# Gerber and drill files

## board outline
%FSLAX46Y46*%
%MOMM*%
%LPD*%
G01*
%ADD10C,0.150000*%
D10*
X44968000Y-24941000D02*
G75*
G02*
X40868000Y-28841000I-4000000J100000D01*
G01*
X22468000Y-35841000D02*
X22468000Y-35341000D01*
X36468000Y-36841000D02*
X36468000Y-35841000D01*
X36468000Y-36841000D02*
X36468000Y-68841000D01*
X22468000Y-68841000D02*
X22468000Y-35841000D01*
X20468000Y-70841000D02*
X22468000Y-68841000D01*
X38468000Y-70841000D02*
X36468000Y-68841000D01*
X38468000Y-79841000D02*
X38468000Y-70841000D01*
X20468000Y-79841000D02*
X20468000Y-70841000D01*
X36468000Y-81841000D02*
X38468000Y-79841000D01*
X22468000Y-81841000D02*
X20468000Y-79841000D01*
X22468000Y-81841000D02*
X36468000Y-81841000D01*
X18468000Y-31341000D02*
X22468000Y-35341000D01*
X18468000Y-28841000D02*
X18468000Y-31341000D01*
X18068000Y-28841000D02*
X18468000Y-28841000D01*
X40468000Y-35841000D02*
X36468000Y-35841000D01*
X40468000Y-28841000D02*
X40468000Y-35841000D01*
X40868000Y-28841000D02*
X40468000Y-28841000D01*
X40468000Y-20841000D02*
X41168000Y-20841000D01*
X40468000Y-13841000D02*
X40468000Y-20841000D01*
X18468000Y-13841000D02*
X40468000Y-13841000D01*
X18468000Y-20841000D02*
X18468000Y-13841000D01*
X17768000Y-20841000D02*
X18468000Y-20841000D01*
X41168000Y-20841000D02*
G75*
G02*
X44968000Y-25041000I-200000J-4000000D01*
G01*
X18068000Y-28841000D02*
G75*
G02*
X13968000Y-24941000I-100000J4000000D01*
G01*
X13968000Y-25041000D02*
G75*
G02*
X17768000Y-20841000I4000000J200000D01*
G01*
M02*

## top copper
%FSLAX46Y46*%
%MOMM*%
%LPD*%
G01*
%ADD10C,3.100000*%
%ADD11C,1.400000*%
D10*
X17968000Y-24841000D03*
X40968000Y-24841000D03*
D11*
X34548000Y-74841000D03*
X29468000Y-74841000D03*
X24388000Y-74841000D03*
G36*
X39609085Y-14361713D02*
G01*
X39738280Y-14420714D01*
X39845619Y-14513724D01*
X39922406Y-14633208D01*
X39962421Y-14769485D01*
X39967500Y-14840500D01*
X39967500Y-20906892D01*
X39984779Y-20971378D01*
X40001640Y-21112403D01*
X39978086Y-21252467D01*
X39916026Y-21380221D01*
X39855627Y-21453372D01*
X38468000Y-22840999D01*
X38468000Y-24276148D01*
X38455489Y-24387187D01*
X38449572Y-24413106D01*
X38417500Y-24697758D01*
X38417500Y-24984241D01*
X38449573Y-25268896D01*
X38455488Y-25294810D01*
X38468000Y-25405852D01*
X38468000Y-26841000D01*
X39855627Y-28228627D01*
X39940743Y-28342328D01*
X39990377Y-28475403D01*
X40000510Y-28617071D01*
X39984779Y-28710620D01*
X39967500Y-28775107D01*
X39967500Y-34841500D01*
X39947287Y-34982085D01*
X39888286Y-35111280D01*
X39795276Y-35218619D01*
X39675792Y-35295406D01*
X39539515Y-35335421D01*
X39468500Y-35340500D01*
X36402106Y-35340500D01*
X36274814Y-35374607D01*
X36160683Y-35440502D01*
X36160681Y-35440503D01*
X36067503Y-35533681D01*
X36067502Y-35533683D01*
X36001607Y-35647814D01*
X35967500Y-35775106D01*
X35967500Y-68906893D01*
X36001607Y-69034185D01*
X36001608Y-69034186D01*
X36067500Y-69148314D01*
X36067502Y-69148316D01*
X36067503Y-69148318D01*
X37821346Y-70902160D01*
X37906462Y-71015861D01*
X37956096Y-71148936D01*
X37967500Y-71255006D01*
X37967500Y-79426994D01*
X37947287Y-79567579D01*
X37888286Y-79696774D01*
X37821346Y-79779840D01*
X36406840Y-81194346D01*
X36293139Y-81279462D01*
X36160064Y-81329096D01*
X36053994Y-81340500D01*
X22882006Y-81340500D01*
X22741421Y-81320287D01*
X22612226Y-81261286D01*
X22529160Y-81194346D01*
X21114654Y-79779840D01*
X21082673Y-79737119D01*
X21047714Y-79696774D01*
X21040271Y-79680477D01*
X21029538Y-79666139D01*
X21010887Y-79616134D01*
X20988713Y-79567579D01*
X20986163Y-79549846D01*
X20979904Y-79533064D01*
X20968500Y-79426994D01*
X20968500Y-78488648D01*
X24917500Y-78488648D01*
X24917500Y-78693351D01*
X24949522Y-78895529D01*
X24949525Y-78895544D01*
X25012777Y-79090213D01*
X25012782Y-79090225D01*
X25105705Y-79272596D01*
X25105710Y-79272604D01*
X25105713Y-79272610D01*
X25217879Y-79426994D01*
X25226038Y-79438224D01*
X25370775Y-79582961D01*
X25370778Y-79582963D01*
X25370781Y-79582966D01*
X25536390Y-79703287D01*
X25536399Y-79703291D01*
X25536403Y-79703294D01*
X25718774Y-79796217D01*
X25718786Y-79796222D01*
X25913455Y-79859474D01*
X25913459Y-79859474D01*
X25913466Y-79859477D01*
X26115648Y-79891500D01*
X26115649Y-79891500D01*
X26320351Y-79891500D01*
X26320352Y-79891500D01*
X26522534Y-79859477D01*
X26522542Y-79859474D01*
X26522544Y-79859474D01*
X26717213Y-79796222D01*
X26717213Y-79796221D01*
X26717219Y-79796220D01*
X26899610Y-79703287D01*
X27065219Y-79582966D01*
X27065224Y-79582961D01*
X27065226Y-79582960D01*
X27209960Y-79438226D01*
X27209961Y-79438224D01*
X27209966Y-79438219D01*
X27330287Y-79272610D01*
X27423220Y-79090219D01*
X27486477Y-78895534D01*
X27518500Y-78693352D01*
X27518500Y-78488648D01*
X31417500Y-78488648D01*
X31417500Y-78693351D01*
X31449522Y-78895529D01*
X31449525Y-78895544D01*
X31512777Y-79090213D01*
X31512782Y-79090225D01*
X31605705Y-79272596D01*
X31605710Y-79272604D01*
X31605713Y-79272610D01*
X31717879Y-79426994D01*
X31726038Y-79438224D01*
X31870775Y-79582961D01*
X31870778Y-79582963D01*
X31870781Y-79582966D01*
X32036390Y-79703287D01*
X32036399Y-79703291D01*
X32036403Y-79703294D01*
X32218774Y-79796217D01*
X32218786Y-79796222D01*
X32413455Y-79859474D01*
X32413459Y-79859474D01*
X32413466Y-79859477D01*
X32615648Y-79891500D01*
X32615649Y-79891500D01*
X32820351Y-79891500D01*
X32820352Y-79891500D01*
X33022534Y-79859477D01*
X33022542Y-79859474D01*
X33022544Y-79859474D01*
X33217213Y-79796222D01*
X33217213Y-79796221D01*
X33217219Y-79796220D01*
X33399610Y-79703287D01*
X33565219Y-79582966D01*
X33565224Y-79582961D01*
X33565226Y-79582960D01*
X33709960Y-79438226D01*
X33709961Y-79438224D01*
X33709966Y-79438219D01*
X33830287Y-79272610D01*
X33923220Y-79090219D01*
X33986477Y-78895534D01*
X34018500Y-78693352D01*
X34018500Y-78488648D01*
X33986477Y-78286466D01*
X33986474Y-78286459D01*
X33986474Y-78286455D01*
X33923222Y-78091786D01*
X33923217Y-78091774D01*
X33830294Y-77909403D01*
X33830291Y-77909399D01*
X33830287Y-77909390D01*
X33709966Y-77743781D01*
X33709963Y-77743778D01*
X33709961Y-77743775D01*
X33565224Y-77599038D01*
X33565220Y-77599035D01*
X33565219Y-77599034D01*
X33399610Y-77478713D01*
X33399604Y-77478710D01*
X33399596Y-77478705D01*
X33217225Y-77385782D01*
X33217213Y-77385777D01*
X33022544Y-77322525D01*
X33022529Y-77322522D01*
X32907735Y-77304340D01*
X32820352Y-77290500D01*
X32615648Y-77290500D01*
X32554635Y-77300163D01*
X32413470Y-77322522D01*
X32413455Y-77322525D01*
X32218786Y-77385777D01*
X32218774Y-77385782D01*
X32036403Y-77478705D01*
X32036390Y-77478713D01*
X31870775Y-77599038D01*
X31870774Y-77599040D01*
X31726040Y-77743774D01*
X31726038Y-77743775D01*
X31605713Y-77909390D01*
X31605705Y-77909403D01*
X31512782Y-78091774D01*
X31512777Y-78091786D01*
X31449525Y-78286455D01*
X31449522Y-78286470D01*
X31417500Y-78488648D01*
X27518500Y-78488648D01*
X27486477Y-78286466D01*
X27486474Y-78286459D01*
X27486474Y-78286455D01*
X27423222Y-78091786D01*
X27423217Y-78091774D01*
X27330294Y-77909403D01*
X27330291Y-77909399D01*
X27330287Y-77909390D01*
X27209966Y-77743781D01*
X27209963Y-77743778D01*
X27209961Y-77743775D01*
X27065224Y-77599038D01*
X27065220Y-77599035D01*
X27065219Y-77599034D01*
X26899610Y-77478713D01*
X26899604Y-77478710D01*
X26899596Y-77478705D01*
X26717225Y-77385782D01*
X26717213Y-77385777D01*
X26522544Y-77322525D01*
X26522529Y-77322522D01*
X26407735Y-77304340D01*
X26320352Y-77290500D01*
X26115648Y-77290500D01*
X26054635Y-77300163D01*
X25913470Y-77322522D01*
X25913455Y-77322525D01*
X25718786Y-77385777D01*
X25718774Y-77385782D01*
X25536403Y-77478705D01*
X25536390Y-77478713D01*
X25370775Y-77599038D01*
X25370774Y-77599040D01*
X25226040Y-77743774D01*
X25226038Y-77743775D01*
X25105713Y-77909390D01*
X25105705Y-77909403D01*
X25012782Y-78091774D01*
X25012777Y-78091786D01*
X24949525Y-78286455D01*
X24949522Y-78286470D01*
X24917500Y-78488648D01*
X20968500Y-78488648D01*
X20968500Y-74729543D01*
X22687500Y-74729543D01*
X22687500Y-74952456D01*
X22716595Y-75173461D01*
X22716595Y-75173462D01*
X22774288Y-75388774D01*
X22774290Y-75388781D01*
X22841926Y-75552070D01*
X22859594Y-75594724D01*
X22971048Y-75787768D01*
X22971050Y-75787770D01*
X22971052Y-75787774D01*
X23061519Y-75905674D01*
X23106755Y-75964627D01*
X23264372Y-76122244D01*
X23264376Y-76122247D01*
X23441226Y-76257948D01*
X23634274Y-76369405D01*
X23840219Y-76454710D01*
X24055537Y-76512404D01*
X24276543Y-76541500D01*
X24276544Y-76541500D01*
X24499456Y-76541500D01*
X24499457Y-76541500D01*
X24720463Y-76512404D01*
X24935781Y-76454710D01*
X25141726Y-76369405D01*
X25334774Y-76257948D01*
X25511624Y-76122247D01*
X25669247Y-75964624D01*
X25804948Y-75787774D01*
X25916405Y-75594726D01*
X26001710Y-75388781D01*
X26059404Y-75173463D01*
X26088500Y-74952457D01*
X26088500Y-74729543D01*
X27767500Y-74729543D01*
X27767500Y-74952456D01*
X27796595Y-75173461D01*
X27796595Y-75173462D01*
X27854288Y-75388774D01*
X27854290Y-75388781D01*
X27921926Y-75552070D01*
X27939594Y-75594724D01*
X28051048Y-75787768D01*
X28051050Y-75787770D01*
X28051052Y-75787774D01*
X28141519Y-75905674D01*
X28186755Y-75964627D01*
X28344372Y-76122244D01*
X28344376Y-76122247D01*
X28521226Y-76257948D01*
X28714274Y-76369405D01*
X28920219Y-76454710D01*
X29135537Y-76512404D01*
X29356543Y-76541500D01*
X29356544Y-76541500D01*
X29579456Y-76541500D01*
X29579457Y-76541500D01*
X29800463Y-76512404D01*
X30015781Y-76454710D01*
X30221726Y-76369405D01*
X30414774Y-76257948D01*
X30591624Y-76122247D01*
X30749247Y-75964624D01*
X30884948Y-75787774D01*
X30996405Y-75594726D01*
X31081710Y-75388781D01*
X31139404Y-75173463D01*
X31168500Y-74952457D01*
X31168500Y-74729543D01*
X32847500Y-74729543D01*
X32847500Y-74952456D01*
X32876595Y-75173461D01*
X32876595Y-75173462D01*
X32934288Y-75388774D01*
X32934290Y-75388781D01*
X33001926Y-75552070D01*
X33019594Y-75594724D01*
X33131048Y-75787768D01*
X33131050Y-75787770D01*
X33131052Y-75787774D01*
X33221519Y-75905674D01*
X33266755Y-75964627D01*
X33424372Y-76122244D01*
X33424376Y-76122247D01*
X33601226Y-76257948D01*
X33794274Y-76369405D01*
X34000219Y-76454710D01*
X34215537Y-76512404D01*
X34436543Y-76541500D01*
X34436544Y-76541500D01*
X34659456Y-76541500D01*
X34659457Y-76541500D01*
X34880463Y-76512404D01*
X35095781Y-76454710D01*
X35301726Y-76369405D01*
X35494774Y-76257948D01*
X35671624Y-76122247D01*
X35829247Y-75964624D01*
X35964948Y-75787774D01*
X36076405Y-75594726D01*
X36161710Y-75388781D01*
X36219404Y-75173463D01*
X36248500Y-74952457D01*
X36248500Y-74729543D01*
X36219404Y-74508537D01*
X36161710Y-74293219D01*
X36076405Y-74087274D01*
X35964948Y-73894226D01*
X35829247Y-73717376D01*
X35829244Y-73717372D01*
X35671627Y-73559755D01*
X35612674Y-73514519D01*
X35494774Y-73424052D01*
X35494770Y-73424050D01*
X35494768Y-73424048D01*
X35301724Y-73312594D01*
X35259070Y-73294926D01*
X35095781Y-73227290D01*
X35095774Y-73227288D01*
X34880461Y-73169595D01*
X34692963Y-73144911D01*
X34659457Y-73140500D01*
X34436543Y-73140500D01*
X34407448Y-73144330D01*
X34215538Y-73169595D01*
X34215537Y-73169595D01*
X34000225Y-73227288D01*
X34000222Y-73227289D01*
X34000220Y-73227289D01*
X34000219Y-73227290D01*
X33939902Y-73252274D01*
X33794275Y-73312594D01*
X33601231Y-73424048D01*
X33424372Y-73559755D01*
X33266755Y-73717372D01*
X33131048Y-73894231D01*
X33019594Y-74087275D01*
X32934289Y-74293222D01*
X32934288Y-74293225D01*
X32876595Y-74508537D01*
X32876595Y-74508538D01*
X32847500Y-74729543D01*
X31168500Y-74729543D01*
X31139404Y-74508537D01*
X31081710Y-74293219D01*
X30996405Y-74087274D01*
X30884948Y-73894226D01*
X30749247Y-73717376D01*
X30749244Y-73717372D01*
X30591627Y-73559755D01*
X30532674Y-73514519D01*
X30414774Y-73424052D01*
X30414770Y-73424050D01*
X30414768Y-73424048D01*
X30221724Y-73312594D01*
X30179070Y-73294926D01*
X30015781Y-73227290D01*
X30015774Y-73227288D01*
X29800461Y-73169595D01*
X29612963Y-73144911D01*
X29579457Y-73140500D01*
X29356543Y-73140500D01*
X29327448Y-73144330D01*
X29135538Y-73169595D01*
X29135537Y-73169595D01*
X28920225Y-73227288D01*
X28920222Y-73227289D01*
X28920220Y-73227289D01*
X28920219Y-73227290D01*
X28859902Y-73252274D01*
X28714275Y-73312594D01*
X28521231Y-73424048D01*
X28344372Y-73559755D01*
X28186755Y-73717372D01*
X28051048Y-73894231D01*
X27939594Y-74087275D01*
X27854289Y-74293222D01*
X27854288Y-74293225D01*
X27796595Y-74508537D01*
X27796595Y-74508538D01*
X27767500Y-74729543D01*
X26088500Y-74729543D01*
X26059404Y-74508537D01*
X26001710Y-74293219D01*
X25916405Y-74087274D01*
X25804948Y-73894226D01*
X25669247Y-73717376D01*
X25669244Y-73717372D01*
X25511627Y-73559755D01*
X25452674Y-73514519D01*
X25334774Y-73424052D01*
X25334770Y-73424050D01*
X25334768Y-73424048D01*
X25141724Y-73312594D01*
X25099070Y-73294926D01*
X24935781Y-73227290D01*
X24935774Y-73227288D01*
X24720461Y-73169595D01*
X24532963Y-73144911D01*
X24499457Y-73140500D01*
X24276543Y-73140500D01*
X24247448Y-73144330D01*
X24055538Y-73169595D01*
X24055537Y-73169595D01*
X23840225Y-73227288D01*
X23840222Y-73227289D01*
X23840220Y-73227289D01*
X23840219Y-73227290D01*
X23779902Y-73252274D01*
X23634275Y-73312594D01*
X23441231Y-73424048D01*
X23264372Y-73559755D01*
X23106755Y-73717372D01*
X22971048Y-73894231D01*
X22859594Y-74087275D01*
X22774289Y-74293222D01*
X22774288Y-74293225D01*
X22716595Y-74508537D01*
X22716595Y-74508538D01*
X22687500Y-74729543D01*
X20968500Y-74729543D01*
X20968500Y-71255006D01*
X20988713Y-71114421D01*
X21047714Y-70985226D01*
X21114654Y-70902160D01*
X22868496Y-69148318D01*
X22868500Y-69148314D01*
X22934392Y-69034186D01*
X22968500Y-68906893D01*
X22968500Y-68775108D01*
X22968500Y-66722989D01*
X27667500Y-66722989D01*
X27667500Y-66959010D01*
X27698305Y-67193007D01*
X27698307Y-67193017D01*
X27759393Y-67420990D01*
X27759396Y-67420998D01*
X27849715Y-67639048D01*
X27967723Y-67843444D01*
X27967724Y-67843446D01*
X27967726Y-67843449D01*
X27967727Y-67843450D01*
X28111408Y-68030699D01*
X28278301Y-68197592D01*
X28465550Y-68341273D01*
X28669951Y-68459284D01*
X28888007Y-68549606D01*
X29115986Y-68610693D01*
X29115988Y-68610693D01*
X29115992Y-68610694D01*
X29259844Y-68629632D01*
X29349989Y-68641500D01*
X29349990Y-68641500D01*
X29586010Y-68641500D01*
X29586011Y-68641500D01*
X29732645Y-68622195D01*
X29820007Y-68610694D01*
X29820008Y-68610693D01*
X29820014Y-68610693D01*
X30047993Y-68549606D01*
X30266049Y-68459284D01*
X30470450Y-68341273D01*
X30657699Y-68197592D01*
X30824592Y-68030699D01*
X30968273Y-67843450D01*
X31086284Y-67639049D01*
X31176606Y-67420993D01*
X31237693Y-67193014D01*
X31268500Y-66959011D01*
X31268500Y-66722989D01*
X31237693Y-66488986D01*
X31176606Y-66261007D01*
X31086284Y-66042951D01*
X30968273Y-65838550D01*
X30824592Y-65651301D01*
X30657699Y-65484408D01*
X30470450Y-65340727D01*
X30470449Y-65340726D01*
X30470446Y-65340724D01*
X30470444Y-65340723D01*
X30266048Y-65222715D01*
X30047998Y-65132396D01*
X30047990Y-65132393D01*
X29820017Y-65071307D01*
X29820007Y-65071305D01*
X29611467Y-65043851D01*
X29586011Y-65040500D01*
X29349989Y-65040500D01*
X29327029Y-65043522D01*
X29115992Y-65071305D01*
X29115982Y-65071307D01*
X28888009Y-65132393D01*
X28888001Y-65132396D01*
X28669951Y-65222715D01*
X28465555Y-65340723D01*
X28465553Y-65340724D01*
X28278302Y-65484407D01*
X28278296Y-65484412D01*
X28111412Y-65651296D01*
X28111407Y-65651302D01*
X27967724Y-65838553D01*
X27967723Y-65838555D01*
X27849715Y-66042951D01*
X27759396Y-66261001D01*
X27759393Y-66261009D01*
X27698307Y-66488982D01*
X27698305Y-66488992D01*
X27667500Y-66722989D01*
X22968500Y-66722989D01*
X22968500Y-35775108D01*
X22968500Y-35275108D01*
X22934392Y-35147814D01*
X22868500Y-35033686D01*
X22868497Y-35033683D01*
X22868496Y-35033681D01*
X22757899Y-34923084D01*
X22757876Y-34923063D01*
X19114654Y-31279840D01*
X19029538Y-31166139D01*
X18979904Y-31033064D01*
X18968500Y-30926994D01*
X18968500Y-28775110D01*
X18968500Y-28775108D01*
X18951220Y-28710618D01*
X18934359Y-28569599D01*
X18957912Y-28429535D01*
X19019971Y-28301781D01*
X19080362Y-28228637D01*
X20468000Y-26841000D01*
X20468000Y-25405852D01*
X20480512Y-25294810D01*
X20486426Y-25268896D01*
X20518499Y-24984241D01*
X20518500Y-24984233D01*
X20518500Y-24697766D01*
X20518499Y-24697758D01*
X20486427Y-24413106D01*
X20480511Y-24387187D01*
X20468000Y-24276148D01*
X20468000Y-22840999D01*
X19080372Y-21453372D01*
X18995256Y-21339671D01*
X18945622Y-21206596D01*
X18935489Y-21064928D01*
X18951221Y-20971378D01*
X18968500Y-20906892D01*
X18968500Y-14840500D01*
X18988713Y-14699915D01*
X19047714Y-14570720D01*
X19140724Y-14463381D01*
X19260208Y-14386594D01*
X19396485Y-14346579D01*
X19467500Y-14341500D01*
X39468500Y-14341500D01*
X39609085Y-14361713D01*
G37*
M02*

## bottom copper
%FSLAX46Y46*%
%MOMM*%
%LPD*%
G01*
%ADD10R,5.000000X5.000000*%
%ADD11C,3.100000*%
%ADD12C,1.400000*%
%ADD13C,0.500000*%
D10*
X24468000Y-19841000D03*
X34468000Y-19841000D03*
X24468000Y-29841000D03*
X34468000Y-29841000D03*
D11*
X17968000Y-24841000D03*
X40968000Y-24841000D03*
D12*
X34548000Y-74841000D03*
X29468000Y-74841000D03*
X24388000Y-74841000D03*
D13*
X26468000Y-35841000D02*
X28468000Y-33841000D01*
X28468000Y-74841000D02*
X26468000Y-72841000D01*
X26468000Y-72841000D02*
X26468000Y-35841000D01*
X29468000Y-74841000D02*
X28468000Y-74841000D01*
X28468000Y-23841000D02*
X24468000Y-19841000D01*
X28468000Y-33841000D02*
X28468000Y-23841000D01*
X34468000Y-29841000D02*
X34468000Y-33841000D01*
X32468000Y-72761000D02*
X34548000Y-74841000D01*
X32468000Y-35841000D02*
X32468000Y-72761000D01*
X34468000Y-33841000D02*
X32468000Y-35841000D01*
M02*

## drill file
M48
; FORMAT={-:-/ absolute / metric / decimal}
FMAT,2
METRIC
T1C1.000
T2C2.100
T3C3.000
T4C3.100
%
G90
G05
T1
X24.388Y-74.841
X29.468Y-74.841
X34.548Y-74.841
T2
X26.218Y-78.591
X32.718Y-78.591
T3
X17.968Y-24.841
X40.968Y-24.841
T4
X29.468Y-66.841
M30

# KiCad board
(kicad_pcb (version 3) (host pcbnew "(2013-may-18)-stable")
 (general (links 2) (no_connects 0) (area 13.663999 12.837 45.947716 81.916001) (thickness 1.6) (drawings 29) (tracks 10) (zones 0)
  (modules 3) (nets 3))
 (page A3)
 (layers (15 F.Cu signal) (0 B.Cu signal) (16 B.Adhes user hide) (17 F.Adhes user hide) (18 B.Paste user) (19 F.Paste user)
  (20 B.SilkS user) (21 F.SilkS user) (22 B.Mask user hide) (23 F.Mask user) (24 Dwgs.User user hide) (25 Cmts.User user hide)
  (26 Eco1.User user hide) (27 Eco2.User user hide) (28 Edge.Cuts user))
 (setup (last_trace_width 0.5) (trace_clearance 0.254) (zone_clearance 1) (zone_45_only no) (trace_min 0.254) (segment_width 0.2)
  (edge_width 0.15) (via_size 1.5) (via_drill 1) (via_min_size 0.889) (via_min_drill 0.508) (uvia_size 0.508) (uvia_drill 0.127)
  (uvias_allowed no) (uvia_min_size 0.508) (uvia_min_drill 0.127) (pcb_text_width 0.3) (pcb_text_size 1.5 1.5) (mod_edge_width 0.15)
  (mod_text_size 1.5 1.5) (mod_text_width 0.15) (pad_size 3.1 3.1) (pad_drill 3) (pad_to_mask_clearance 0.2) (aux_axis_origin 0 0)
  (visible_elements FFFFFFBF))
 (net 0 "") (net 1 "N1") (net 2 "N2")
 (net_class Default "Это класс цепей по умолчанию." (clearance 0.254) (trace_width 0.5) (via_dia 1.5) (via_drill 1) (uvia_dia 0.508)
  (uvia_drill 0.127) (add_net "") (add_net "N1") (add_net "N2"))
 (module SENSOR (layer B.Cu) (at 17.968 13.341)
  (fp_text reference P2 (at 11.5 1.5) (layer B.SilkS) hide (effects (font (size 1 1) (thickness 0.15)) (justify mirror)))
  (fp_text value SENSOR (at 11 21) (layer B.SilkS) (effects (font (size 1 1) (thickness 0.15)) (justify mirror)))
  (pad 2 smd rect (at 6.5 6.5) (size 5 5) (layers B.Cu B.Mask) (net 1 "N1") (solder_mask_margin 0.1))
  (pad 3 smd rect (at 16.5 6.5) (size 5 5) (layers B.Cu B.Mask))
  (pad 1 smd rect (at 6.5 16.5) (size 5 5) (layers B.Cu B.Mask))
  (pad 4 smd rect (at 16.5 16.5) (size 5 5) (layers B.Cu B.Mask) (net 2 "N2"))
  (pad "" np_thru_hole circle (at 0 11.5) (size 3.1 3.1) (drill 3) (layers *.Cu *.Mask B.SilkS))
  (pad "" np_thru_hole circle (at 23 11.5) (size 3.1 3.1) (drill 3) (layers *.Cu *.Mask B.SilkS)))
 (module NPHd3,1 (layer F.Cu) (at 29.468 66.841)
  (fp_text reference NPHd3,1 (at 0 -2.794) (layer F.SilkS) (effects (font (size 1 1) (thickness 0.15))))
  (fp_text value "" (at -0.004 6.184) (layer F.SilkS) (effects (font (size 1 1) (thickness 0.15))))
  (pad "" np_thru_hole circle (at 0 0) (size 3.1 3.1) (drill 3.1) (layers *.Cu *.Mask F.SilkS)))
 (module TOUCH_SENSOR (layer F.Cu) (at 29.468 74.841 180)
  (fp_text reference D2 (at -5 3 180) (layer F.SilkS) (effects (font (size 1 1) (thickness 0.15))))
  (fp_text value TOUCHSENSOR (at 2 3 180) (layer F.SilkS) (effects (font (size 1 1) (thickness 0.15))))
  (pad 2 thru_hole circle (at -5.08 0 180) (size 1.4 1.4) (drill 1) (layers *.Cu *.Mask F.SilkS) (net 2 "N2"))
  (pad 1 thru_hole circle (at 0 0 180) (size 1.4 1.4) (drill 1) (layers *.Cu *.Mask F.SilkS) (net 1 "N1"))
  (pad 3 thru_hole circle (at 5.08 0 180) (size 1.4 1.4) (drill 1) (layers *.Cu *.Mask F.SilkS))
  (pad "" np_thru_hole circle (at -3.25 -3.75 180) (size 2.1 2.1) (drill 2.1) (layers *.Cu *.Mask F.SilkS))
  (pad "" np_thru_hole circle (at 3.25 -3.75 180) (size 2.1 2.1) (drill 2.1) (layers *.Cu *.Mask F.SilkS)))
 (gr_arc (start 40.968 24.841) (end 44.968 24.941) (angle 90) (layer Edge.Cuts) (width 0.15))
 (gr_line (start 22.468 35.841) (end 22.468 35.341) (angle 90) (layer Edge.Cuts) (width 0.15))
 (gr_line (start 36.468 36.841) (end 36.468 35.841) (angle 90) (layer Edge.Cuts) (width 0.15))
 (gr_line (start 36.468 36.841) (end 36.468 68.841) (angle 90) (layer Edge.Cuts) (width 0.15))
 (gr_line (start 22.468 68.841) (end 22.468 35.841) (angle 90) (layer Edge.Cuts) (width 0.15))
 (gr_line (start 20.468 70.841) (end 22.468 68.841) (angle 90) (layer Edge.Cuts) (width 0.15))
 (gr_line (start 38.468 70.841) (end 36.468 68.841) (angle 90) (layer Edge.Cuts) (width 0.15))
 (gr_line (start 38.468 79.841) (end 38.468 70.841) (angle 90) (layer Edge.Cuts) (width 0.15))
 (gr_line (start 20.468 79.841) (end 20.468 70.841) (angle 90) (layer Edge.Cuts) (width 0.15))
 (gr_line (start 36.468 81.841) (end 38.468 79.841) (angle 90) (layer Edge.Cuts) (width 0.15))
 (gr_line (start 22.468 81.841) (end 20.468 79.841) (angle 90) (layer Edge.Cuts) (width 0.15))
 (gr_line (start 22.468 81.841) (end 36.468 81.841) (angle 90) (layer Edge.Cuts) (width 0.15))
 (gr_line (start 18.468 31.341) (end 22.468 35.341) (angle 90) (layer Edge.Cuts) (width 0.15))
 (gr_line (start 18.468 28.841) (end 18.468 31.341) (angle 90) (layer Edge.Cuts) (width 0.15))
 (gr_line (start 18.068 28.841) (end 18.468 28.841) (angle 90) (layer Edge.Cuts) (width 0.15))
 (gr_line (start 40.468 35.841) (end 36.468 35.841) (angle 90) (layer Edge.Cuts) (width 0.15))
 (gr_line (start 40.468 28.841) (end 40.468 35.841) (angle 90) (layer Edge.Cuts) (width 0.15))
 (gr_line (start 40.868 28.841) (end 40.468 28.841) (angle 90) (layer Edge.Cuts) (width 0.15))
 (gr_line (start 40.468 20.841) (end 41.168 20.841) (angle 90) (layer Edge.Cuts) (width 0.15))
 (gr_line (start 40.468 13.841) (end 40.468 20.841) (angle 90) (layer Edge.Cuts) (width 0.15))
 (gr_line (start 18.468 13.841) (end 40.468 13.841) (angle 90) (layer Edge.Cuts) (width 0.15))
 (gr_line (start 18.468 20.841) (end 18.468 13.841) (angle 90) (layer Edge.Cuts) (width 0.15))
 (gr_line (start 17.768 20.841) (end 18.468 20.841) (angle 90) (layer Edge.Cuts) (width 0.15))
 (gr_arc (start 40.968 24.841) (end 41.168 20.841) (angle 90) (layer Edge.Cuts) (width 0.15))
 (gr_arc (start 17.968 24.841) (end 18.068 28.841) (angle 90) (layer Edge.Cuts) (width 0.15))
 (gr_arc (start 17.968 24.841) (end 13.968 25.041) (angle 90) (layer Edge.Cuts) (width 0.15))
 (segment (start 26.468 35.841) (end 28.468 33.841) (width 0.5) (layer B.Cu) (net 1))
 (segment (start 28.468 74.841) (end 26.468 72.841) (width 0.5) (layer B.Cu) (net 1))
 (segment (start 26.468 72.841) (end 26.468 35.841) (width 0.5) (layer B.Cu) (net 1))
 (segment (start 29.468 74.841) (end 28.468 74.841) (width 0.5) (layer B.Cu) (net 1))
 (segment (start 28.468 23.841) (end 24.468 19.841) (width 0.5) (layer B.Cu) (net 1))
 (segment (start 28.468 33.841) (end 28.468 23.841) (width 0.5) (layer B.Cu) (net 1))
 (segment (start 34.468 29.841) (end 34.468 33.841) (width 0.5) (layer B.Cu) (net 2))
 (segment (start 32.468 72.761) (end 34.548 74.841) (width 0.5) (layer B.Cu) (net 2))
 (segment (start 32.468 35.841) (end 32.468 72.761) (width 0.5) (layer B.Cu) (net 2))
 (segment (start 34.468 33.841) (end 32.468 35.841) (width 0.5) (layer B.Cu) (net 2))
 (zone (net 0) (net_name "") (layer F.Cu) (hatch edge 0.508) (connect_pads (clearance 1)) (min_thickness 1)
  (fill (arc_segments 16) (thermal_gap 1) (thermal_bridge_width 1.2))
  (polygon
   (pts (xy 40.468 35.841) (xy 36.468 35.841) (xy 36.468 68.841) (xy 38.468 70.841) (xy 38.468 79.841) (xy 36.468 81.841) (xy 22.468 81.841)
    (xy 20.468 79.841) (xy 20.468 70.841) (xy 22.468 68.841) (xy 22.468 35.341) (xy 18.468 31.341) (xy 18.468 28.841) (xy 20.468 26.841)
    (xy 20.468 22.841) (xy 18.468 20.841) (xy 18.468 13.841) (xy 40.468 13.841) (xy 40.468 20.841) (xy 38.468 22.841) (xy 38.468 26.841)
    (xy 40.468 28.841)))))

